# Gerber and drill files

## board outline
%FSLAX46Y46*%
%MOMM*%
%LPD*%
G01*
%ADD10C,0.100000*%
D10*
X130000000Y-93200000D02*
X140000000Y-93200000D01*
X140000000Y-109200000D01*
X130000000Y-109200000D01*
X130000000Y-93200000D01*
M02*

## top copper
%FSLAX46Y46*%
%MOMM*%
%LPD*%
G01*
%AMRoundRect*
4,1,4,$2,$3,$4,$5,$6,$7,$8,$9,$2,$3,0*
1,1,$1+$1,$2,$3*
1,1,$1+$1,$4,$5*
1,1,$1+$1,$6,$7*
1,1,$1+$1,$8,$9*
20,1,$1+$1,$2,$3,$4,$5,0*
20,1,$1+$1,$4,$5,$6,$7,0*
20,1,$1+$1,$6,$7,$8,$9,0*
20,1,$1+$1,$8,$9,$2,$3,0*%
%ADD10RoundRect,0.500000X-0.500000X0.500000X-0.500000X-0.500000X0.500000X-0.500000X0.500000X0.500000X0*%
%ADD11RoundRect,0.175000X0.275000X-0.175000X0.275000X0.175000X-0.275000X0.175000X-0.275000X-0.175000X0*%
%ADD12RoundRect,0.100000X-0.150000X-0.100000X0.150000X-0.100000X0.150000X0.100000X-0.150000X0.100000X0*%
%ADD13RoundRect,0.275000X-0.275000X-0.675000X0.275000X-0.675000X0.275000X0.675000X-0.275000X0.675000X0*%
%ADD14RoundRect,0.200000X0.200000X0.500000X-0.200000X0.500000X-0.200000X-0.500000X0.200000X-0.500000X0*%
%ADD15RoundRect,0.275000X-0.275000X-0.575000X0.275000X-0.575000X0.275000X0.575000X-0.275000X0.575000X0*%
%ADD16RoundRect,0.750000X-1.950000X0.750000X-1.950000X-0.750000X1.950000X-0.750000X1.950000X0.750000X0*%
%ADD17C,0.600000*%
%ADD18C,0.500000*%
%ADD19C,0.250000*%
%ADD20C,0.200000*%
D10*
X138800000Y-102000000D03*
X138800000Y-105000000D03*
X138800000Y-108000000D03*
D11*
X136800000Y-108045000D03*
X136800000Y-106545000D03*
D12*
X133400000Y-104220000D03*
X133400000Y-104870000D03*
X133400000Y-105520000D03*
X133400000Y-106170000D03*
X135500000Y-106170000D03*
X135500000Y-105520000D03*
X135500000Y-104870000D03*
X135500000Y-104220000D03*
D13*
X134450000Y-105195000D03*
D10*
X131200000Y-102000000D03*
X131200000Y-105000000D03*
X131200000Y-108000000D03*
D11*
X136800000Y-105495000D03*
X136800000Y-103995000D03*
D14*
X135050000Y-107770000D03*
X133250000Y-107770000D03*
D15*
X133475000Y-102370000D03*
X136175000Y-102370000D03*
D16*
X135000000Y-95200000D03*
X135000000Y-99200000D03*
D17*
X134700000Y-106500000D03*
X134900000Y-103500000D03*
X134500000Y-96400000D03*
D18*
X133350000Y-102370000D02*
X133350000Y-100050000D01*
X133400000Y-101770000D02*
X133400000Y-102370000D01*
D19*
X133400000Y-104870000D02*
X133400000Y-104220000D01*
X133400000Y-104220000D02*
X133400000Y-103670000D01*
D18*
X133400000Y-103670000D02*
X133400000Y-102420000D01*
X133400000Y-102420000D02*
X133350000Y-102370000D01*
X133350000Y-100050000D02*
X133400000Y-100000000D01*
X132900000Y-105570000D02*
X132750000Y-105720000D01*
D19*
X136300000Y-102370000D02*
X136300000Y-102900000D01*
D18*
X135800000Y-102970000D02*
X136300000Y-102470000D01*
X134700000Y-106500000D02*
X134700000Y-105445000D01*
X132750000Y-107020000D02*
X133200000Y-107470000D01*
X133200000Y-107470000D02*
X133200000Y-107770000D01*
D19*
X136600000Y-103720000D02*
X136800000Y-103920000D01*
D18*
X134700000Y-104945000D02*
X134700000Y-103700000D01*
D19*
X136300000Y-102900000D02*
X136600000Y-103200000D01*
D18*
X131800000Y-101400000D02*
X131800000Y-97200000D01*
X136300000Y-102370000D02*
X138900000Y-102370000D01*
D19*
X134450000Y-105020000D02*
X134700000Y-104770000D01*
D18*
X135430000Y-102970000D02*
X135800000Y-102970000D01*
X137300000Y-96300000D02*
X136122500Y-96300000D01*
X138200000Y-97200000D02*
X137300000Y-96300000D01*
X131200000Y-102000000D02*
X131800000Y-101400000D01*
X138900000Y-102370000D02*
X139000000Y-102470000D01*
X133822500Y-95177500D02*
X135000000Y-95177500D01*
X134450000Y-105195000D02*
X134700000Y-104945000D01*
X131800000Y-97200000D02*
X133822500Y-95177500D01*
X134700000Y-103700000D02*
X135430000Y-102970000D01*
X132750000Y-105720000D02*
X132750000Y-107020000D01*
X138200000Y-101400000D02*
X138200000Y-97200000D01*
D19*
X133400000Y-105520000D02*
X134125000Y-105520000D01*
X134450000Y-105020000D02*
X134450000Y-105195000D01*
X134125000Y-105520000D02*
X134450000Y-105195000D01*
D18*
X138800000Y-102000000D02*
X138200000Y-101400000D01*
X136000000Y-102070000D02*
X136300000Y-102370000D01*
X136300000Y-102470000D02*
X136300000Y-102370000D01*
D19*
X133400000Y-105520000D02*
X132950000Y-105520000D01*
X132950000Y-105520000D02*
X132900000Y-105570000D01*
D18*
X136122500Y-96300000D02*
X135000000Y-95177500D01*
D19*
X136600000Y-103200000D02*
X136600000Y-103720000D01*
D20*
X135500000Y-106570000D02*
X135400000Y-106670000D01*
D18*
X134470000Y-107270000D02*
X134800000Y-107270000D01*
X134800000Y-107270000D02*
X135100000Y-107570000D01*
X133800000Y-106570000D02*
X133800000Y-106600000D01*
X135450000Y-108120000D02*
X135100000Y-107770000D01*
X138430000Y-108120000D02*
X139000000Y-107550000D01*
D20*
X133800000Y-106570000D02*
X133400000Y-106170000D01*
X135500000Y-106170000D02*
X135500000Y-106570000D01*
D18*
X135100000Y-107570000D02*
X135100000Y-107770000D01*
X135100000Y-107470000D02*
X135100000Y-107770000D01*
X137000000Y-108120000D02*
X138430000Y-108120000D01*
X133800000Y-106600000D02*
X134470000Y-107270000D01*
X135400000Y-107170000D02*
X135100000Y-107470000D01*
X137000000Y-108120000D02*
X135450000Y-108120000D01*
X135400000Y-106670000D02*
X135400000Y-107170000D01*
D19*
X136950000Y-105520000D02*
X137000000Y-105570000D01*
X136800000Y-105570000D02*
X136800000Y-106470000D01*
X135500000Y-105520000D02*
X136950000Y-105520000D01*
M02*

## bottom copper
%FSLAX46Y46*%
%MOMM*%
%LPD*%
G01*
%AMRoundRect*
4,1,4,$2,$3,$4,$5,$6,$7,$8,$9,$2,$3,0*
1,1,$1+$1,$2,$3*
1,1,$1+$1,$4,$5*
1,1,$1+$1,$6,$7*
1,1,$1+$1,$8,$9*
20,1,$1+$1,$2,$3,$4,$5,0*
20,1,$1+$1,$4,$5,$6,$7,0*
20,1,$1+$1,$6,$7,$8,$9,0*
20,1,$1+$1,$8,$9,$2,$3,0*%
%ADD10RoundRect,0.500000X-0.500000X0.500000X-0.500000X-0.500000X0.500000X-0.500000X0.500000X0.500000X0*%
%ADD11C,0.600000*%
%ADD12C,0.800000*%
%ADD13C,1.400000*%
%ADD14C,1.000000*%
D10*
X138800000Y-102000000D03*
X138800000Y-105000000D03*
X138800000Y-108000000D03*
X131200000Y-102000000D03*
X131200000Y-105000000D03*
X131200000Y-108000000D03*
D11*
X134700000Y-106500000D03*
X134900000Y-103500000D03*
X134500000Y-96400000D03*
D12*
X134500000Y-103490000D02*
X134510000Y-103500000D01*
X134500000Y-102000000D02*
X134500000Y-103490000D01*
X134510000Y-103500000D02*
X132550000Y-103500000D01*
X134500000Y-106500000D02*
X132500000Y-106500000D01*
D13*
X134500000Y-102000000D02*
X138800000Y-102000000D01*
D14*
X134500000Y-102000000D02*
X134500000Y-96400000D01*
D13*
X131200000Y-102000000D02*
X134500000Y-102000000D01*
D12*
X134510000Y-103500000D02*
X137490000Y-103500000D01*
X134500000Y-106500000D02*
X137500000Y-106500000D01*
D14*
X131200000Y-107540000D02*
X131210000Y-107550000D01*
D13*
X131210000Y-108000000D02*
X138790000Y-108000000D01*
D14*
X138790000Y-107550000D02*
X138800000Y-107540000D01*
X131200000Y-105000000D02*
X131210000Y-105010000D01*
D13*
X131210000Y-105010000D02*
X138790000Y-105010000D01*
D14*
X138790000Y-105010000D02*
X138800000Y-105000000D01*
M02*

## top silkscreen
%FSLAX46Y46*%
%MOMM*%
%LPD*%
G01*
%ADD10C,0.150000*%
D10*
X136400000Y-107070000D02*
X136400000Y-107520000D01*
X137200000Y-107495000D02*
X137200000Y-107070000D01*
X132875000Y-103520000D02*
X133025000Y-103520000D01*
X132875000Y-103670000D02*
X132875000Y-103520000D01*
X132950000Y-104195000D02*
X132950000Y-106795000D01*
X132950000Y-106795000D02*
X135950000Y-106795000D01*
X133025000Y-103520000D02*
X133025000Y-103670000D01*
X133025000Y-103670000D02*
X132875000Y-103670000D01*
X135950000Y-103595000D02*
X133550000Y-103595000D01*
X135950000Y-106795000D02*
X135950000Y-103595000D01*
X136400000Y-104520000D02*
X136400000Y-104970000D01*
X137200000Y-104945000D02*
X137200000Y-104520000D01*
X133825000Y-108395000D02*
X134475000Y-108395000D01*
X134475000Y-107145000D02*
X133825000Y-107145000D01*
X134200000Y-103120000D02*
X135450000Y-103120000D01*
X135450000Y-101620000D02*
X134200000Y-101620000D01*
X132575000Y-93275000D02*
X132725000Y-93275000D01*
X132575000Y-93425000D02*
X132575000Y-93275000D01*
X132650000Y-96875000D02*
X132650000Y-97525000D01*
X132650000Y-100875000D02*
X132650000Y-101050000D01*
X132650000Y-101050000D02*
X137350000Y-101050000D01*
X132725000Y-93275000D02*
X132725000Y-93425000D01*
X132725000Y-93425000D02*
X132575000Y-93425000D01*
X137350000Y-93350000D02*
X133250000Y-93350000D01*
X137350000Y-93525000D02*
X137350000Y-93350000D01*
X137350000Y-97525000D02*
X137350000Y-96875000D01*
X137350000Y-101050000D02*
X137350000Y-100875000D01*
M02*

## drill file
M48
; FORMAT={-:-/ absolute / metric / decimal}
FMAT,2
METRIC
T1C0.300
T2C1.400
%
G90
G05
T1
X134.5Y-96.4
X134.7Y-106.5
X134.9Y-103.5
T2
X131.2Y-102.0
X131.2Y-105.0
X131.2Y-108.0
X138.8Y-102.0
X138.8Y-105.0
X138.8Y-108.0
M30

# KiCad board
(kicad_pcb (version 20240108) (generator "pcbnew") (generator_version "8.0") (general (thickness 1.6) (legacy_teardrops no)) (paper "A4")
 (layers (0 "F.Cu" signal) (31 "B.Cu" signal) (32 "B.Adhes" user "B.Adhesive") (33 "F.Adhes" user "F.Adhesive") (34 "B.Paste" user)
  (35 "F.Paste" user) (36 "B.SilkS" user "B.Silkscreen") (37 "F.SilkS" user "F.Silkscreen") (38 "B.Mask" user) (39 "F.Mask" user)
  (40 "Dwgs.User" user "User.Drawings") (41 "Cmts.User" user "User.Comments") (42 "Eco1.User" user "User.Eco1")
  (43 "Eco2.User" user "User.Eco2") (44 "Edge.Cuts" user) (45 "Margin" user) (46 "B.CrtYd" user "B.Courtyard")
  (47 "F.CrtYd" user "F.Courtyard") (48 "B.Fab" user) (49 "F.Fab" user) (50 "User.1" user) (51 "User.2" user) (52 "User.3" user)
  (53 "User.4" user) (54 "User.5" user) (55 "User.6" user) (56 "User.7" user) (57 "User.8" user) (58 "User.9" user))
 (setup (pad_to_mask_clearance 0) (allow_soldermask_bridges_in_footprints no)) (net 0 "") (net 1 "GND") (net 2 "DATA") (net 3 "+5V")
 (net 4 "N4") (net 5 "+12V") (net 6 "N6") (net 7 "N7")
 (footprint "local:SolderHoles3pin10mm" (layer "F.Cu") (at 138.8 105 -90)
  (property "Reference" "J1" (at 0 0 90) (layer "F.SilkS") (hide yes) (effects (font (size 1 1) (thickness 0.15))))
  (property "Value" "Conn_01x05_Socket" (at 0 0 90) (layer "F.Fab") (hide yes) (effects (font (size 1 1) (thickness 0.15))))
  (pad "1" thru_hole roundrect (at -3 0 270) (size 2 2) (drill 1.4) (layers "*.Cu" "*.Mask") (remove_unused_layers yes)
   (keep_end_layers yes) (zone_layer_connections) (roundrect_rratio 0.25) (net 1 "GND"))
  (pad "2" thru_hole roundrect (at 0 0 270) (size 2 2) (drill 1.4) (layers "*.Cu" "*.Mask") (remove_unused_layers yes) (keep_end_layers yes)
   (zone_layer_connections) (roundrect_rratio 0.25) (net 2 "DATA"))
  (pad "3" thru_hole roundrect (at 3 0 270) (size 2 2) (drill 1.4) (layers "*.Cu" "*.Mask") (remove_unused_layers yes) (keep_end_layers yes)
   (zone_layer_connections) (roundrect_rratio 0.25) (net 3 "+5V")))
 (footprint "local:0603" (layer "F.Cu") (at 136.8 107.295 90)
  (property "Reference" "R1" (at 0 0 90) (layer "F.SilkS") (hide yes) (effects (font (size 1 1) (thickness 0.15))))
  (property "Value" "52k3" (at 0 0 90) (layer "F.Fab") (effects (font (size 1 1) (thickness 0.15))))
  (fp_line (start 0.225 -0.4) (end -0.225 -0.4) (stroke (width 0.15) (type solid)) (layer "F.SilkS"))
  (fp_line (start -0.2 0.4) (end 0.225 0.4) (stroke (width 0.15) (type solid)) (layer "F.SilkS"))
  (pad "1" smd roundrect (at -0.75 0 90) (size 0.7 0.9) (layers "F.Cu" "F.Paste" "F.Mask") (roundrect_rratio 0.25) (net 3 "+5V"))
  (pad "2" smd roundrect (at 0.75 0 90) (size 0.7 0.9) (layers "F.Cu" "F.Paste" "F.Mask") (roundrect_rratio 0.25) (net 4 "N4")))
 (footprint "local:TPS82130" (layer "F.Cu") (at 134.45 105.195)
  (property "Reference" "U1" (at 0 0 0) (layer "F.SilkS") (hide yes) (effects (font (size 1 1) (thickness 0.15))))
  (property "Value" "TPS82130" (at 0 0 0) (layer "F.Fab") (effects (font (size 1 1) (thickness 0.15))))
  (fp_line (start -1.575 -1.675) (end -1.425 -1.675) (stroke (width 0.15) (type solid)) (layer "F.SilkS"))
  (fp_line (start -1.575 -1.525) (end -1.575 -1.675) (stroke (width 0.15) (type solid)) (layer "F.SilkS"))
  (fp_line (start -1.5 -1) (end -1.5 1.6) (stroke (width 0.15) (type solid)) (layer "F.SilkS"))
  (fp_line (start -1.5 1.6) (end 1.5 1.6) (stroke (width 0.15) (type solid)) (layer "F.SilkS"))
  (fp_line (start -1.425 -1.675) (end -1.425 -1.525) (stroke (width 0.15) (type solid)) (layer "F.SilkS"))
  (fp_line (start -1.425 -1.525) (end -1.575 -1.525) (stroke (width 0.15) (type solid)) (layer "F.SilkS"))
  (fp_line (start 1.5 -1.6) (end -0.9 -1.6) (stroke (width 0.15) (type solid)) (layer "F.SilkS"))
  (fp_line (start 1.5 1.6) (end 1.5 -1.6) (stroke (width 0.15) (type solid)) (layer "F.SilkS"))
  (pad "1" smd roundrect (at -1.05 -0.975) (size 0.5 0.4) (layers "F.Cu" "F.Paste" "F.Mask") (roundrect_rratio 0.25) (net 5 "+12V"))
  (pad "2" smd roundrect (at -1.05 -0.325) (size 0.5 0.4) (layers "F.Cu" "F.Paste" "F.Mask") (roundrect_rratio 0.25) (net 5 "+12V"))
  (pad "3" smd roundrect (at -1.05 0.325) (size 0.5 0.4) (layers "F.Cu" "F.Paste" "F.Mask") (roundrect_rratio 0.25) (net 1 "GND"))
  (pad "4" smd roundrect (at -1.05 0.975) (size 0.5 0.4) (layers "F.Cu" "F.Paste" "F.Mask") (roundrect_rratio 0.25) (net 3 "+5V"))
  (pad "5" smd roundrect (at 1.05 0.975) (size 0.5 0.4) (layers "F.Cu" "F.Paste" "F.Mask") (roundrect_rratio 0.25) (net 3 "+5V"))
  (pad "6" smd roundrect (at 1.05 0.325) (size 0.5 0.4) (layers "F.Cu" "F.Paste" "F.Mask") (roundrect_rratio 0.25) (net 4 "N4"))
  (pad "7" smd roundrect (at 1.05 -0.325) (size 0.5 0.4) (layers "F.Cu" "F.Paste" "F.Mask") (roundrect_rratio 0.25) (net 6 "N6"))
  (pad "8" smd roundrect (at 1.05 -0.975) (size 0.5 0.4) (layers "F.Cu" "F.Paste" "F.Mask") (roundrect_rratio 0.25) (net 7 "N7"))
  (pad "9" smd roundrect (at 0 0) (size 1.1 1.9) (layers "F.Cu" "F.Paste" "F.Mask") (roundrect_rratio 0.25) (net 1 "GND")))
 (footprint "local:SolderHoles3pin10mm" (layer "F.Cu") (at 131.2 105 -90)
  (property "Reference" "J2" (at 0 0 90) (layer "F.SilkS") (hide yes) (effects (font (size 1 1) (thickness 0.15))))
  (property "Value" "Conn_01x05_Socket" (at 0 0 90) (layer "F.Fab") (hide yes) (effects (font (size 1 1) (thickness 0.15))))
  (pad "1" thru_hole roundrect (at -3 0 270) (size 2 2) (drill 1.4) (layers "*.Cu" "*.Mask") (remove_unused_layers yes)
   (keep_end_layers yes) (zone_layer_connections) (roundrect_rratio 0.25) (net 1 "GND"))
  (pad "2" thru_hole roundrect (at 0 0 270) (size 2 2) (drill 1.4) (layers "*.Cu" "*.Mask") (remove_unused_layers yes) (keep_end_layers yes)
   (zone_layer_connections) (roundrect_rratio 0.25) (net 2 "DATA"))
  (pad "3" thru_hole roundrect (at 3 0 270) (size 2 2) (drill 1.4) (layers "*.Cu" "*.Mask") (remove_unused_layers yes) (keep_end_layers yes)
   (zone_layer_connections) (roundrect_rratio 0.25) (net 3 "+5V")))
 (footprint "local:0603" (layer "F.Cu") (at 136.8 104.745 90)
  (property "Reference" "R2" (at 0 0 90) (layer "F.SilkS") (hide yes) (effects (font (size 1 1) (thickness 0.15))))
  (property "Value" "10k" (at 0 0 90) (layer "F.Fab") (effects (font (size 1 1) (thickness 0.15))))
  (fp_line (start 0.225 -0.4) (end -0.225 -0.4) (stroke (width 0.15) (type solid)) (layer "F.SilkS"))
  (fp_line (start -0.2 0.4) (end 0.225 0.4) (stroke (width 0.15) (type solid)) (layer "F.SilkS"))
  (pad "1" smd roundrect (at -0.75 0 90) (size 0.7 0.9) (layers "F.Cu" "F.Paste" "F.Mask") (roundrect_rratio 0.25) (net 4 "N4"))
  (pad "2" smd roundrect (at 0.75 0 90) (size 0.7 0.9) (layers "F.Cu" "F.Paste" "F.Mask") (roundrect_rratio 0.25) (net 1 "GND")))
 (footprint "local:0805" (layer "F.Cu") (at 134.15 107.77 180)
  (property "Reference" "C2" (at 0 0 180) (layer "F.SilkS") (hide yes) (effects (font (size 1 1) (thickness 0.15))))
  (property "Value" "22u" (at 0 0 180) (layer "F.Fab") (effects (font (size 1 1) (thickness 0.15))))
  (fp_line (start 0.325 -0.625) (end -0.325 -0.625) (stroke (width 0.15) (type solid)) (layer "F.SilkS"))
  (fp_line (start -0.325 0.625) (end 0.325 0.625) (stroke (width 0.15) (type solid)) (layer "F.SilkS"))
  (pad "1" smd roundrect (at -0.9 0 180) (size 0.8 1.4) (layers "F.Cu" "F.Paste" "F.Mask") (roundrect_rratio 0.25) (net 3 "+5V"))
  (pad "2" smd roundrect (at 0.9 0 180) (size 0.8 1.4) (layers "F.Cu" "F.Paste" "F.Mask") (roundrect_rratio 0.25) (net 1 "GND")))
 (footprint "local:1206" (layer "F.Cu") (at 134.825 102.37)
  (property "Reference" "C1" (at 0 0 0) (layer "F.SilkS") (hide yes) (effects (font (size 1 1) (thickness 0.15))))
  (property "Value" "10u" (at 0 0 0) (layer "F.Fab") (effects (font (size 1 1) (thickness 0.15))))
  (fp_line (start -0.625 0.75) (end 0.625 0.75) (stroke (width 0.15) (type solid)) (layer "F.SilkS"))
  (fp_line (start 0.625 -0.75) (end -0.625 -0.75) (stroke (width 0.15) (type solid)) (layer "F.SilkS"))
  (pad "1" smd roundrect (at -1.35 0) (size 1.1 1.7) (layers "F.Cu" "F.Paste" "F.Mask") (roundrect_rratio 0.25) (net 5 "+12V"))
  (pad "2" smd roundrect (at 1.35 0) (size 1.1 1.7) (layers "F.Cu" "F.Paste" "F.Mask") (roundrect_rratio 0.25) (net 1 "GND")))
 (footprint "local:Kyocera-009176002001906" (layer "F.Cu") (at 135 97.2 -90)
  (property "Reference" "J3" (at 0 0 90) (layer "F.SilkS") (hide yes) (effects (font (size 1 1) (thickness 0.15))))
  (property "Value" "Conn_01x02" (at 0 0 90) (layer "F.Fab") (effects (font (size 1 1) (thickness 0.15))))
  (fp_line (start -3.925 2.425) (end -3.925 2.275) (stroke (width 0.15) (type solid)) (layer "F.SilkS"))
  (fp_line (start -3.775 2.425) (end -3.925 2.425) (stroke (width 0.15) (type solid)) (layer "F.SilkS"))
  (fp_line (start -0.325 2.35) (end 0.325 2.35) (stroke (width 0.15) (type solid)) (layer "F.SilkS"))
  (fp_line (start 3.675 2.35) (end 3.85 2.35) (stroke (width 0.15) (type solid)) (layer "F.SilkS"))
  (fp_line (start 3.85 2.35) (end 3.85 -2.35) (stroke (width 0.15) (type solid)) (layer "F.SilkS"))
  (fp_line (start -3.925 2.275) (end -3.775 2.275) (stroke (width 0.15) (type solid)) (layer "F.SilkS"))
  (fp_line (start -3.775 2.275) (end -3.775 2.425) (stroke (width 0.15) (type solid)) (layer "F.SilkS"))
  (fp_line (start -3.85 -2.35) (end -3.85 1.75) (stroke (width 0.15) (type solid)) (layer "F.SilkS"))
  (fp_line (start -3.675 -2.35) (end -3.85 -2.35) (stroke (width 0.15) (type solid)) (layer "F.SilkS"))
  (fp_line (start 0.325 -2.35) (end -0.325 -2.35) (stroke (width 0.15) (type solid)) (layer "F.SilkS"))
  (fp_line (start 3.85 -2.35) (end 3.675 -2.35) (stroke (width 0.15) (type solid)) (layer "F.SilkS"))
  (pad "1" smd roundrect (at -2 0 270) (size 3 5.4) (layers "F.Cu" "F.Paste" "F.Mask") (roundrect_rratio 0.25) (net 1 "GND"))
  (pad "2" smd roundrect (at 2 0 270) (size 3 5.4) (layers "F.Cu" "F.Paste" "F.Mask") (roundrect_rratio 0.25) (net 5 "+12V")))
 (gr_rect (start 130 93.2) (end 140 109.2) (stroke (width 0.1) (type default)) (fill none) (layer "Edge.Cuts"))
 (segment (start 133.35 102.37) (end 133.35 100.05) (width 0.5) (layer "F.Cu") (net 5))
 (segment (start 133.4 101.77) (end 133.4 102.37) (width 0.5) (layer "F.Cu") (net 5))
 (segment (start 133.4 104.87) (end 133.4 104.22) (width 0.25) (layer "F.Cu") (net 5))
 (segment (start 133.4 104.22) (end 133.4 103.67) (width 0.25) (layer "F.Cu") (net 5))
 (segment (start 133.4 103.67) (end 133.4 102.42) (width 0.5) (layer "F.Cu") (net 5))
 (segment (start 133.4 102.42) (end 133.35 102.37) (width 0.5) (layer "F.Cu") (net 5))
 (segment (start 133.35 100.05) (end 133.4 100) (width 0.5) (layer "F.Cu") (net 5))
 (segment (start 132.9 105.57) (end 132.75 105.72) (width 0.5) (layer "F.Cu") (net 1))
 (segment (start 136.3 102.37) (end 136.3 102.9) (width 0.25) (layer "F.Cu") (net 1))
 (segment (start 135.8 102.97) (end 136.3 102.47) (width 0.5) (layer "F.Cu") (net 1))
 (segment (start 134.7 106.5) (end 134.7 105.445) (width 0.5) (layer "F.Cu") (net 1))
 (segment (start 132.75 107.02) (end 133.2 107.47) (width 0.5) (layer "F.Cu") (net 1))
 (segment (start 133.2 107.47) (end 133.2 107.77) (width 0.5) (layer "F.Cu") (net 1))
 (segment (start 136.6 103.72) (end 136.8 103.92) (width 0.25) (layer "F.Cu") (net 1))
 (segment (start 134.7 104.945) (end 134.7 103.7) (width 0.5) (layer "F.Cu") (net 1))
 (segment (start 136.3 102.9) (end 136.6 103.2) (width 0.25) (layer "F.Cu") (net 1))
 (segment (start 131.8 101.4) (end 131.8 97.2) (width 0.5) (layer "F.Cu") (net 1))
 (segment (start 136.3 102.37) (end 138.9 102.37) (width 0.5) (layer "F.Cu") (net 1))
 (segment (start 134.45 105.02) (end 134.7 104.77) (width 0.25) (layer "F.Cu") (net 1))
 (segment (start 135.43 102.97) (end 135.8 102.97) (width 0.5) (layer "F.Cu") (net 1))
 (segment (start 137.3 96.3) (end 136.1225 96.3) (width 0.5) (layer "F.Cu") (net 1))
 (segment (start 138.2 97.2) (end 137.3 96.3) (width 0.5) (layer "F.Cu") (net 1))
 (segment (start 131.2 102) (end 131.8 101.4) (width 0.5) (layer "F.Cu") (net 1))
 (segment (start 138.9 102.37) (end 139 102.47) (width 0.5) (layer "F.Cu") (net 1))
 (segment (start 133.8225 95.1775) (end 135 95.1775) (width 0.5) (layer "F.Cu") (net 1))
 (segment (start 134.45 105.195) (end 134.7 104.945) (width 0.5) (layer "F.Cu") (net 1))
 (segment (start 131.8 97.2) (end 133.8225 95.1775) (width 0.5) (layer "F.Cu") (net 1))
 (segment (start 134.7 103.7) (end 135.43 102.97) (width 0.5) (layer "F.Cu") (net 1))
 (segment (start 132.75 105.72) (end 132.75 107.02) (width 0.5) (layer "F.Cu") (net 1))
 (segment (start 138.2 101.4) (end 138.2 97.2) (width 0.5) (layer "F.Cu") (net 1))
 (segment (start 133.4 105.52) (end 134.125 105.52) (width 0.25) (layer "F.Cu") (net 1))
 (segment (start 134.45 105.02) (end 134.45 105.195) (width 0.25) (layer "F.Cu") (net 1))
 (segment (start 134.125 105.52) (end 134.45 105.195) (width 0.25) (layer "F.Cu") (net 1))
 (segment (start 138.8 102) (end 138.2 101.4) (width 0.5) (layer "F.Cu") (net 1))
 (segment (start 136 102.07) (end 136.3 102.37) (width 0.5) (layer "F.Cu") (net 1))
 (segment (start 136.3 102.47) (end 136.3 102.37) (width 0.5) (layer "F.Cu") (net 1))
 (segment (start 133.4 105.52) (end 132.95 105.52) (width 0.25) (layer "F.Cu") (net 1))
 (segment (start 132.95 105.52) (end 132.9 105.57) (width 0.25) (layer "F.Cu") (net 1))
 (segment (start 136.1225 96.3) (end 135 95.1775) (width 0.5) (layer "F.Cu") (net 1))
 (segment (start 136.6 103.2) (end 136.6 103.72) (width 0.25) (layer "F.Cu") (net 1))
 (via (at 134.7 106.5) (size 0.6) (drill 0.3) (layers "F.Cu" "B.Cu") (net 1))
 (via (at 134.9 103.5) (size 0.6) (drill 0.3) (layers "F.Cu" "B.Cu") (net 1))
 (via (at 134.5 96.4) (size 0.6) (drill 0.3) (layers "F.Cu" "B.Cu") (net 1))
 (segment (start 134.5 103.49) (end 134.51 103.5) (width 0.8) (layer "B.Cu") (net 1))
 (segment (start 134.5 102) (end 134.5 103.49) (width 0.8) (layer "B.Cu") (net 1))
 (segment (start 134.51 103.5) (end 132.55 103.5) (width 0.8) (layer "B.Cu") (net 1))
 (segment (start 134.5 106.5) (end 132.5 106.5) (width 0.8) (layer "B.Cu") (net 1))
 (segment (start 134.5 102) (end 138.8 102) (width 1.4) (layer "B.Cu") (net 1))
 (segment (start 134.5 102) (end 134.5 96.4) (width 1) (layer "B.Cu") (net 1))
 (segment (start 131.2 102) (end 134.5 102) (width 1.4) (layer "B.Cu") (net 1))
 (segment (start 134.51 103.5) (end 137.49 103.5) (width 0.8) (layer "B.Cu") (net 1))
 (segment (start 134.5 106.5) (end 137.5 106.5) (width 0.8) (layer "B.Cu") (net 1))
 (segment (start 135.5 106.57) (end 135.4 106.67) (width 0.2) (layer "F.Cu") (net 3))
 (segment (start 134.47 107.27) (end 134.8 107.27) (width 0.5) (layer "F.Cu") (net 3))
 (segment (start 134.8 107.27) (end 135.1 107.57) (width 0.5) (layer "F.Cu") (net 3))
 (segment (start 133.8 106.57) (end 133.8 106.6) (width 0.5) (layer "F.Cu") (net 3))
 (segment (start 135.45 108.12) (end 135.1 107.77) (width 0.5) (layer "F.Cu") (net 3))
 (segment (start 138.43 108.12) (end 139 107.55) (width 0.5) (layer "F.Cu") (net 3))
 (segment (start 133.8 106.57) (end 133.4 106.17) (width 0.2) (layer "F.Cu") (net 3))
 (segment (start 135.5 106.17) (end 135.5 106.57) (width 0.2) (layer "F.Cu") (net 3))
 (segment (start 135.1 107.57) (end 135.1 107.77) (width 0.5) (layer "F.Cu") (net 3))
 (segment (start 135.1 107.47) (end 135.1 107.77) (width 0.5) (layer "F.Cu") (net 3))
 (segment (start 137 108.12) (end 138.43 108.12) (width 0.5) (layer "F.Cu") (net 3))
 (segment (start 133.8 106.6) (end 134.47 107.27) (width 0.5) (layer "F.Cu") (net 3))
 (segment (start 135.4 107.17) (end 135.1 107.47) (width 0.5) (layer "F.Cu") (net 3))
 (segment (start 137 108.12) (end 135.45 108.12) (width 0.5) (layer "F.Cu") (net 3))
 (segment (start 135.4 106.67) (end 135.4 107.17) (width 0.5) (layer "F.Cu") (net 3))
 (segment (start 131.2 107.54) (end 131.21 107.55) (width 1) (layer "B.Cu") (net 3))
 (segment (start 131.21 108) (end 138.79 108) (width 1.4) (layer "B.Cu") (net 3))
 (segment (start 138.79 107.55) (end 138.8 107.54) (width 1) (layer "B.Cu") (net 3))
 (segment (start 136.95 105.52) (end 137 105.57) (width 0.25) (layer "F.Cu") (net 4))
 (segment (start 136.8 105.57) (end 136.8 106.47) (width 0.25) (layer "F.Cu") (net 4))
 (segment (start 135.5 105.52) (end 136.95 105.52) (width 0.25) (layer "F.Cu") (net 4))
 (segment (start 131.2 105) (end 131.21 105.01) (width 1) (layer "B.Cu") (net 2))
 (segment (start 131.21 105.01) (end 138.79 105.01) (width 1.4) (layer "B.Cu") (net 2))
 (segment (start 138.79 105.01) (end 138.8 105) (width 1) (layer "B.Cu") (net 2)))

